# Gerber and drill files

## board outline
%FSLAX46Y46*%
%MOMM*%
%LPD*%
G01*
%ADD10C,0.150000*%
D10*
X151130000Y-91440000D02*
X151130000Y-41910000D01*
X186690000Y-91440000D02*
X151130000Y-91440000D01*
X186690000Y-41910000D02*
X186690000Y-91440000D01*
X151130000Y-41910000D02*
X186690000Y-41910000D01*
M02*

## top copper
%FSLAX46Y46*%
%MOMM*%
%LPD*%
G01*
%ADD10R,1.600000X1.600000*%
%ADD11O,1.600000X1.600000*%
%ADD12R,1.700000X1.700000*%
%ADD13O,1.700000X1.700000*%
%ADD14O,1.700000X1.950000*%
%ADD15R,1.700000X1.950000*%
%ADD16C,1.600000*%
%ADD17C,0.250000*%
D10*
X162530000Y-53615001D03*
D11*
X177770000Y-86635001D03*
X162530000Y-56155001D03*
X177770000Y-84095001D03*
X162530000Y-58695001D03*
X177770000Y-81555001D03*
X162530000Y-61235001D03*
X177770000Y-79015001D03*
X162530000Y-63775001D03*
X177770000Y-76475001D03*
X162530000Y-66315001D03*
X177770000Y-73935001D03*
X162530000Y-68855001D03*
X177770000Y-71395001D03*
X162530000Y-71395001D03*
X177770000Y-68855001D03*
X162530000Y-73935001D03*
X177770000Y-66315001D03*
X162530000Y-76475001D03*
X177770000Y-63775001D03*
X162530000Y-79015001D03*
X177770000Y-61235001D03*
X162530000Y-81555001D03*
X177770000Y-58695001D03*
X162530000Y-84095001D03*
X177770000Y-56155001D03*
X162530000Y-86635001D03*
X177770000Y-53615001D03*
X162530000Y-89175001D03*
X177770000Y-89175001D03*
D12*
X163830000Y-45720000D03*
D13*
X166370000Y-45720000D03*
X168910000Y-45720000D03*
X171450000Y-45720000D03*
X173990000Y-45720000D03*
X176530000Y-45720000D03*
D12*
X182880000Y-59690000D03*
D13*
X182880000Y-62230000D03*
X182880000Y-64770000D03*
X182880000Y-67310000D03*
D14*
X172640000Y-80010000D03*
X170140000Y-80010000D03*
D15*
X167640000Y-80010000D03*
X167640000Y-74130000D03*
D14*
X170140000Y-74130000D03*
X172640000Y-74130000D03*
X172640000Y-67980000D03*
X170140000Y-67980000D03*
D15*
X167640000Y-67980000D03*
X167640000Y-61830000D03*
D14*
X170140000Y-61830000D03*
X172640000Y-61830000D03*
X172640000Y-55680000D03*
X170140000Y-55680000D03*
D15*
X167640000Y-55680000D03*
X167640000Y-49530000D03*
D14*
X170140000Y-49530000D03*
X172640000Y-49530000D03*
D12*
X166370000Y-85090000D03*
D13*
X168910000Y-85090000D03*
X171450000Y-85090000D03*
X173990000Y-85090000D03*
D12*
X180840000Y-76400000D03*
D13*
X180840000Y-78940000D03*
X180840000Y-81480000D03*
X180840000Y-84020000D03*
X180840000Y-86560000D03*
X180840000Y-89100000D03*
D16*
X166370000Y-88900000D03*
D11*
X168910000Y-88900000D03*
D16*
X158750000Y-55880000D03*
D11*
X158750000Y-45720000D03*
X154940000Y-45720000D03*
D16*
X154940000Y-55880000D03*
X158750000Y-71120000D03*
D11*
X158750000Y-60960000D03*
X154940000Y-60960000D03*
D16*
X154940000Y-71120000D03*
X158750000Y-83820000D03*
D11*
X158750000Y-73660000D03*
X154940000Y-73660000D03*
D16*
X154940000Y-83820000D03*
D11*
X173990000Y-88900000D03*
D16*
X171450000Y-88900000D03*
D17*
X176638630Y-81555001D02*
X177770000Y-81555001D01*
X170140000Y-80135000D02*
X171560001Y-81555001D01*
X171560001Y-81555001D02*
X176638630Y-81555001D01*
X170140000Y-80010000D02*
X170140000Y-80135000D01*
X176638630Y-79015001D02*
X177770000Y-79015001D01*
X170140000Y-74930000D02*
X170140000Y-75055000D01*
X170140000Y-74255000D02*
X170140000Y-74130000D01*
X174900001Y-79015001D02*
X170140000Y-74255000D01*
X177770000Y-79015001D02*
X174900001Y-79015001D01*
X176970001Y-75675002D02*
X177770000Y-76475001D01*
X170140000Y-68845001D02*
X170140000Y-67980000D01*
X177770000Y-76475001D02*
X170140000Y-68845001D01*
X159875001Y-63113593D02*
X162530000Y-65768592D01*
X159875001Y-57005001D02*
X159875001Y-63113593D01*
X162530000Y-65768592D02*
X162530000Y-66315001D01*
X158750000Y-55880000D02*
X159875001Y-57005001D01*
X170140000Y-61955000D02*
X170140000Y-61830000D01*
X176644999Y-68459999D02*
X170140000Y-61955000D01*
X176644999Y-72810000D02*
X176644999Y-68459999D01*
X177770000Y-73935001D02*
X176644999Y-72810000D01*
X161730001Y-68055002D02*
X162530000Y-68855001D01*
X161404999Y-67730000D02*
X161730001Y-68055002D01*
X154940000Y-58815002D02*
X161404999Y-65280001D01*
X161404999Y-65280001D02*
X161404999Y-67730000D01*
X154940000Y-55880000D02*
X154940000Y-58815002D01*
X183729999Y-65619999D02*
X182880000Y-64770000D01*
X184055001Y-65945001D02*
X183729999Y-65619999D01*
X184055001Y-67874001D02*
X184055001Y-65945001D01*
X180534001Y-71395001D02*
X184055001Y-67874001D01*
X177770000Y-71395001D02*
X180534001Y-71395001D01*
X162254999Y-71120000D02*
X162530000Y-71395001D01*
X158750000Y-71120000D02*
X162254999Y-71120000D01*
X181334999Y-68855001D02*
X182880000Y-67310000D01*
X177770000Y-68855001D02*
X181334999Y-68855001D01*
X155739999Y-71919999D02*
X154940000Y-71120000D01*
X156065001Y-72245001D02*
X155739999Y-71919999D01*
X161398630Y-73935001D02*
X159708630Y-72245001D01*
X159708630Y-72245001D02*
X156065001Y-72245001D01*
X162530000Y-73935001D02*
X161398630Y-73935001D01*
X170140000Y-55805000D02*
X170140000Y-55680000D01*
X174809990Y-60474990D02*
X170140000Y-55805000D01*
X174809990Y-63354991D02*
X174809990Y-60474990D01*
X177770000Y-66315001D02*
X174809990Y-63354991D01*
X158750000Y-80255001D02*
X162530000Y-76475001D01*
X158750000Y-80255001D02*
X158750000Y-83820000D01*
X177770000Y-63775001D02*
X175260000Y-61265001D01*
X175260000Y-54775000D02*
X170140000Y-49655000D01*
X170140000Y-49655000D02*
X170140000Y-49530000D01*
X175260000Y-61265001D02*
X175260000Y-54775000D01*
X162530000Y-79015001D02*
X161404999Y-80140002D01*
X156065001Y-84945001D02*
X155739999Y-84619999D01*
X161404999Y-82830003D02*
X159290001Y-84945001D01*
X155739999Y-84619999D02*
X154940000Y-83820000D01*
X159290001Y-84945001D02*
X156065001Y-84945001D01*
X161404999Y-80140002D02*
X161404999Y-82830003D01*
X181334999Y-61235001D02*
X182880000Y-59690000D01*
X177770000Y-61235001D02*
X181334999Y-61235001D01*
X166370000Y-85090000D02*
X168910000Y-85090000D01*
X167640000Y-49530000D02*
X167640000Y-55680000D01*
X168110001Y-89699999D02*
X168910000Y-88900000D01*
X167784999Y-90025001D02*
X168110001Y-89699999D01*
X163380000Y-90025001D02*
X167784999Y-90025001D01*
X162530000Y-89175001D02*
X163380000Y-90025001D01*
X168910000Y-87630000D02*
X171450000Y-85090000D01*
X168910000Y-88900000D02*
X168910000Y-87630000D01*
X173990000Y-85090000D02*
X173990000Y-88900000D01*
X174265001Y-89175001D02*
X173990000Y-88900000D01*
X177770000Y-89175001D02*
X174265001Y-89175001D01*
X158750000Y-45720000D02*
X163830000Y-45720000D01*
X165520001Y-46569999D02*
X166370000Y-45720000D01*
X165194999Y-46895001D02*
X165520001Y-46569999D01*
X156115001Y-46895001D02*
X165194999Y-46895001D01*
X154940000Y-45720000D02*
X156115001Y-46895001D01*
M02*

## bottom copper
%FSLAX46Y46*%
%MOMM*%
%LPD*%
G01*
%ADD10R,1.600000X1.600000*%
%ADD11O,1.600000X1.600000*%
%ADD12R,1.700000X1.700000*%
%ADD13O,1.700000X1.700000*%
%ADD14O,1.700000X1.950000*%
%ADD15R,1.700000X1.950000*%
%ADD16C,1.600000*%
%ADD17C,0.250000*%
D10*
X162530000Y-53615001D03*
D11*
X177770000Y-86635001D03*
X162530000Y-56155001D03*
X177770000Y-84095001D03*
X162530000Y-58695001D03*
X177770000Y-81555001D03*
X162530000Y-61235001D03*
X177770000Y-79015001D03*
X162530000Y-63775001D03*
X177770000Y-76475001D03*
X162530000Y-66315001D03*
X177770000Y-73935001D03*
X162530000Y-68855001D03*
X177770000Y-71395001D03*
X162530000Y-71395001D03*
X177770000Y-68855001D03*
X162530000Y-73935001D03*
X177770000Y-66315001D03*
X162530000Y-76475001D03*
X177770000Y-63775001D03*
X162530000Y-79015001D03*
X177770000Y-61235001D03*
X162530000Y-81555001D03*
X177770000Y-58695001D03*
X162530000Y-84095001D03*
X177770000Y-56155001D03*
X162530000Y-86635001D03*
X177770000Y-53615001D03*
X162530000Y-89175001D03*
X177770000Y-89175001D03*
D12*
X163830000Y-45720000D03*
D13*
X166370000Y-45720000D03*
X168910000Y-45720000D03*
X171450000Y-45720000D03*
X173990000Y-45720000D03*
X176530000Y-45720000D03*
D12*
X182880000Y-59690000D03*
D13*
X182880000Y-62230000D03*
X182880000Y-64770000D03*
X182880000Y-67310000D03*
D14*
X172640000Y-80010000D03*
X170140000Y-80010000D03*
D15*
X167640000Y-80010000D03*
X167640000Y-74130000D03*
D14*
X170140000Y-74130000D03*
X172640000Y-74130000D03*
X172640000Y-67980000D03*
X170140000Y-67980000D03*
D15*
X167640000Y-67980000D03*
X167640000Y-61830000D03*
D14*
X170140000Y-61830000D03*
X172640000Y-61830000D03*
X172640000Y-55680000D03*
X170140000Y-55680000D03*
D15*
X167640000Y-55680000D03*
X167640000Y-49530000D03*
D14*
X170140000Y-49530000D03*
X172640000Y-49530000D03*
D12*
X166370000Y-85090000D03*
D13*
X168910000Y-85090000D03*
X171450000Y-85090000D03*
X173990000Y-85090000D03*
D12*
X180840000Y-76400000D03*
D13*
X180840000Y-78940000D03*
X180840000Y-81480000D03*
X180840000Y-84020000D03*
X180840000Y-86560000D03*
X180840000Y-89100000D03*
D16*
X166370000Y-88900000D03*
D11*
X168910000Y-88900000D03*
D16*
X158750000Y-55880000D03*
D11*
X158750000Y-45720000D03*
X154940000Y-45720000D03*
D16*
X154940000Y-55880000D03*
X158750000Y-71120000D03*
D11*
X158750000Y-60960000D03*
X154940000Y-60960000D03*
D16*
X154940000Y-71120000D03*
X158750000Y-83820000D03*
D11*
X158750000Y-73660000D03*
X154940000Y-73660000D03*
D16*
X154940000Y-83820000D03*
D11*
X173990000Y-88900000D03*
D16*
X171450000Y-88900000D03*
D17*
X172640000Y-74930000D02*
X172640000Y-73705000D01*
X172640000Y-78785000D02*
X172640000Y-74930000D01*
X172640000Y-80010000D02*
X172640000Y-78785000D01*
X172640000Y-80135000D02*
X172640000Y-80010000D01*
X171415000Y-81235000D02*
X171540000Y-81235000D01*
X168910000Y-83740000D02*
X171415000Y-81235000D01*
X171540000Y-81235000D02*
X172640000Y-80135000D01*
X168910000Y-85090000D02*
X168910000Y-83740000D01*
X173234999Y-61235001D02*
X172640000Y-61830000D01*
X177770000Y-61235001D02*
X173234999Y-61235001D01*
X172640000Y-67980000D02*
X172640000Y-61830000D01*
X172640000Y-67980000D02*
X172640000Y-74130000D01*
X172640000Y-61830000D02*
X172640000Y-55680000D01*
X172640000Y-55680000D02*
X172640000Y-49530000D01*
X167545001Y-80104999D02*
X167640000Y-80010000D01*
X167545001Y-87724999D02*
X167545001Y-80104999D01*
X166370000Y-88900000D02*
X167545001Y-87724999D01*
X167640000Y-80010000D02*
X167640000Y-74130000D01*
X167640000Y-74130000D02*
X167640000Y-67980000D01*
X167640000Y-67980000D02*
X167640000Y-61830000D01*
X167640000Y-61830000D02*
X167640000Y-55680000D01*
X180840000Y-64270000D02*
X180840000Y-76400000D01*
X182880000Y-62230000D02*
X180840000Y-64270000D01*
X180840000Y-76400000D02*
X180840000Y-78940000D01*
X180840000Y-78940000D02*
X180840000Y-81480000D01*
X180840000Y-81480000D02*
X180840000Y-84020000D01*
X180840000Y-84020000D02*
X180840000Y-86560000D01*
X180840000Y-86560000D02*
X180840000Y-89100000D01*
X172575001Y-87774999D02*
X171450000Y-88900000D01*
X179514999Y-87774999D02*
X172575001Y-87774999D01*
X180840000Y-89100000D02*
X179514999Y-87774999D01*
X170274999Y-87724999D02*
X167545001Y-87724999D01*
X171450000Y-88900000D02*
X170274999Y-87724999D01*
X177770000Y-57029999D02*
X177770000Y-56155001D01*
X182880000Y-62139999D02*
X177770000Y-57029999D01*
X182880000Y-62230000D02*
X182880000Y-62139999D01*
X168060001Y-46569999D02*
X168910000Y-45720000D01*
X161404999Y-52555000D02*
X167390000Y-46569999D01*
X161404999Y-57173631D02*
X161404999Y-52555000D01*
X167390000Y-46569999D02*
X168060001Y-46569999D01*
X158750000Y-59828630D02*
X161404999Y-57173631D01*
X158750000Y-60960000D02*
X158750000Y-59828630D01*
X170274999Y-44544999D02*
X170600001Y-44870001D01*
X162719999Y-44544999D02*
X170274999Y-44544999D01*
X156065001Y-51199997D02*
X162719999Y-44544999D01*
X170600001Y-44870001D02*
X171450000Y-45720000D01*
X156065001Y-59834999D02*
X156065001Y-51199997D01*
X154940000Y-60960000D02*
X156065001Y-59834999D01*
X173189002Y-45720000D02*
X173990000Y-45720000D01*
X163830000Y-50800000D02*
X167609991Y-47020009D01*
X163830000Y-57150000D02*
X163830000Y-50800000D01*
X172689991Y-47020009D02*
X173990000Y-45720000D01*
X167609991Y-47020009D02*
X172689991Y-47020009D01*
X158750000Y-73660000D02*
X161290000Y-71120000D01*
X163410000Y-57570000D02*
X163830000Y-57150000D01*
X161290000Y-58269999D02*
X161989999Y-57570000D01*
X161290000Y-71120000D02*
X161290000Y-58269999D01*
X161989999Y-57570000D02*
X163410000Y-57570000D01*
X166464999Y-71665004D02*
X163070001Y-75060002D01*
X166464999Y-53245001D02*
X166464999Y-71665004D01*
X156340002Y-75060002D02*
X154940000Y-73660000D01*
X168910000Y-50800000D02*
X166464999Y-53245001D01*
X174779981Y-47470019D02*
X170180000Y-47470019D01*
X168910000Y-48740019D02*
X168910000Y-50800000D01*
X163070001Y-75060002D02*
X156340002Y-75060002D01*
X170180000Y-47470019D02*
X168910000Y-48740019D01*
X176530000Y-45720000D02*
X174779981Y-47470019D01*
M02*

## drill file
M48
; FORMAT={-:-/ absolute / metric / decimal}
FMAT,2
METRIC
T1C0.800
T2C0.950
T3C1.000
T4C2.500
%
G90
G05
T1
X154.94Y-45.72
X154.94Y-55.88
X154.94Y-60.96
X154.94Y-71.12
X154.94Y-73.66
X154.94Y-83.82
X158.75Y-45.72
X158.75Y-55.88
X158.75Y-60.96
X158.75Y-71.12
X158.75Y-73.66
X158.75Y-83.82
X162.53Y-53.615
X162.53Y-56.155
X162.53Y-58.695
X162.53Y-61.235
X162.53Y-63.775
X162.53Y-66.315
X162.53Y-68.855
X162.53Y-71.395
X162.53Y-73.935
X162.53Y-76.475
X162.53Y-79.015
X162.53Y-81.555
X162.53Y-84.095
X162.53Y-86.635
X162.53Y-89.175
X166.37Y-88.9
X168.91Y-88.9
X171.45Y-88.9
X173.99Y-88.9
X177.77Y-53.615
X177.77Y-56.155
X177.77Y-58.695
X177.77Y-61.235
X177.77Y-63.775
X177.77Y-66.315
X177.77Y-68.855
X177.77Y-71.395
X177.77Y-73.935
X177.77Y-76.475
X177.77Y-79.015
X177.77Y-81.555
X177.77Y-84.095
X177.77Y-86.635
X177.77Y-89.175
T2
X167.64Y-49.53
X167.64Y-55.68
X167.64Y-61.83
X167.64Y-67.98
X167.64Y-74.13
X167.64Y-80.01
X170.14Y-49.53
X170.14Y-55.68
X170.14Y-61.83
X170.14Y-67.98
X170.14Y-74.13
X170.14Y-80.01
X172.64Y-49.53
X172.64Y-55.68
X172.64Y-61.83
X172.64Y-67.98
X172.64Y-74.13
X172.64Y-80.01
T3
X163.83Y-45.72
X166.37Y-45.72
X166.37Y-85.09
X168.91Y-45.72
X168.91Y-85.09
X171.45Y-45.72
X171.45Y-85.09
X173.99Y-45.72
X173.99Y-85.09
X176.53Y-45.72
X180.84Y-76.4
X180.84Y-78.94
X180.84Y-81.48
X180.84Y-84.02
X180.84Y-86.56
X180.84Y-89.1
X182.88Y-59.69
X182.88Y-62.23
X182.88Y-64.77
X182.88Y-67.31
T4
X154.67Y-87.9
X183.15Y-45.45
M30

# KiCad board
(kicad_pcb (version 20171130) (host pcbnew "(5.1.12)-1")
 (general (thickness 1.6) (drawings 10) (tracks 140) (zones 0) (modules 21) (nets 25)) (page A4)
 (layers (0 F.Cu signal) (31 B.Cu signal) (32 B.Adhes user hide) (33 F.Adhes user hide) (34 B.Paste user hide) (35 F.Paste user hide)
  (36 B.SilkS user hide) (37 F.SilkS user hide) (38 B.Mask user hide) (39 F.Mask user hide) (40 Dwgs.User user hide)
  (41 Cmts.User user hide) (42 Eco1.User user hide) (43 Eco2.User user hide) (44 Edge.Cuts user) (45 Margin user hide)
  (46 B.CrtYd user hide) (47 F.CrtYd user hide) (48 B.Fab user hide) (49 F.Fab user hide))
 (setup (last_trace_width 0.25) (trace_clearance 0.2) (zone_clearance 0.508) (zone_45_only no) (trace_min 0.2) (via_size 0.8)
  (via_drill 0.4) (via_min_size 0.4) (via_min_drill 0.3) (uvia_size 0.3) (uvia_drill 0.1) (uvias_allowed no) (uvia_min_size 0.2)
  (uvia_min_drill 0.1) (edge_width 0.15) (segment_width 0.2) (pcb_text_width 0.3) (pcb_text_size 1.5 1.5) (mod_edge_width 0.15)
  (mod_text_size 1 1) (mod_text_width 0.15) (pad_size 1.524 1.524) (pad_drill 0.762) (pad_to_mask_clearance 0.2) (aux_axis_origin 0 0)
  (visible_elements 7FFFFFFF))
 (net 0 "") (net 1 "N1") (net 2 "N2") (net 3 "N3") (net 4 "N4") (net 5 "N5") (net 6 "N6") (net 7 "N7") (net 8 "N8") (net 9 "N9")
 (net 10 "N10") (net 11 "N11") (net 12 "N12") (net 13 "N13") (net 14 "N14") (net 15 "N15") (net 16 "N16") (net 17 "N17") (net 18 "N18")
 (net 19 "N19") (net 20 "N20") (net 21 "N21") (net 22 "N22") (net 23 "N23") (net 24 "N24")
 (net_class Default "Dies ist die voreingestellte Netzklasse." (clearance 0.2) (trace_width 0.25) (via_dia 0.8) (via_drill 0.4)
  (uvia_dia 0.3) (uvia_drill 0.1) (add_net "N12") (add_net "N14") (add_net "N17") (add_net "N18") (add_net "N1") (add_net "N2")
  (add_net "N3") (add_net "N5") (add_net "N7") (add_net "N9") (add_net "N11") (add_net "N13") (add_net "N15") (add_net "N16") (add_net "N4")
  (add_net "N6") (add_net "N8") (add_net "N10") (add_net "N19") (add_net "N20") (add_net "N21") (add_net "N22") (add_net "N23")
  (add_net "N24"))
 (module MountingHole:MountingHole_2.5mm (layer F.Cu) (at 154.67 87.9)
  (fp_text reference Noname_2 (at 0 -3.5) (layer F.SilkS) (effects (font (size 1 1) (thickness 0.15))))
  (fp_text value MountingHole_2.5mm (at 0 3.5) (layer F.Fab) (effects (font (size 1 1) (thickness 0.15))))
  (pad 1 np_thru_hole circle (at 0 0) (size 2.5 2.5) (drill 2.5) (layers *.Cu *.Mask)))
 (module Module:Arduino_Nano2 (layer F.Cu) (at 162.53 53.615001)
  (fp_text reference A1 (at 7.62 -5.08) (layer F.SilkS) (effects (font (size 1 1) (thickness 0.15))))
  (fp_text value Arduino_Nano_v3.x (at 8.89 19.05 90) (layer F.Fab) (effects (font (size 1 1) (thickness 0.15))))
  (pad 1 thru_hole rect (at 0 0) (size 1.6 1.6) (drill 0.8) (layers *.Cu *.Mask))
  (pad 17 thru_hole oval (at 15.24 33.02) (size 1.6 1.6) (drill 0.8) (layers *.Cu *.Mask))
  (pad 2 thru_hole oval (at 0 2.54) (size 1.6 1.6) (drill 0.8) (layers *.Cu *.Mask))
  (pad 18 thru_hole oval (at 15.24 30.48) (size 1.6 1.6) (drill 0.8) (layers *.Cu *.Mask))
  (pad 3 thru_hole oval (at 0 5.08) (size 1.6 1.6) (drill 0.8) (layers *.Cu *.Mask))
  (pad 19 thru_hole oval (at 15.24 27.94) (size 1.6 1.6) (drill 0.8) (layers *.Cu *.Mask) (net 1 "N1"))
  (pad 4 thru_hole oval (at 0 7.62) (size 1.6 1.6) (drill 0.8) (layers *.Cu *.Mask))
  (pad 20 thru_hole oval (at 15.24 25.4) (size 1.6 1.6) (drill 0.8) (layers *.Cu *.Mask) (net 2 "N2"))
  (pad 5 thru_hole oval (at 0 10.16) (size 1.6 1.6) (drill 0.8) (layers *.Cu *.Mask))
  (pad 21 thru_hole oval (at 15.24 22.86) (size 1.6 1.6) (drill 0.8) (layers *.Cu *.Mask) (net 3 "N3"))
  (pad 6 thru_hole oval (at 0 12.7) (size 1.6 1.6) (drill 0.8) (layers *.Cu *.Mask) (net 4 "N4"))
  (pad 22 thru_hole oval (at 15.24 20.32) (size 1.6 1.6) (drill 0.8) (layers *.Cu *.Mask) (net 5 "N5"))
  (pad 7 thru_hole oval (at 0 15.24) (size 1.6 1.6) (drill 0.8) (layers *.Cu *.Mask) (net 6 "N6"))
  (pad 23 thru_hole oval (at 15.24 17.78) (size 1.6 1.6) (drill 0.8) (layers *.Cu *.Mask) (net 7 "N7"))
  (pad 8 thru_hole oval (at 0 17.78) (size 1.6 1.6) (drill 0.8) (layers *.Cu *.Mask) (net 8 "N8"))
  (pad 24 thru_hole oval (at 15.24 15.24) (size 1.6 1.6) (drill 0.8) (layers *.Cu *.Mask) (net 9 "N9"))
  (pad 9 thru_hole oval (at 0 20.32) (size 1.6 1.6) (drill 0.8) (layers *.Cu *.Mask) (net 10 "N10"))
  (pad 25 thru_hole oval (at 15.24 12.7) (size 1.6 1.6) (drill 0.8) (layers *.Cu *.Mask) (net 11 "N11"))
  (pad 10 thru_hole oval (at 0 22.86) (size 1.6 1.6) (drill 0.8) (layers *.Cu *.Mask) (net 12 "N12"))
  (pad 26 thru_hole oval (at 15.24 10.16) (size 1.6 1.6) (drill 0.8) (layers *.Cu *.Mask) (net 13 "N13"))
  (pad 11 thru_hole oval (at 0 25.4) (size 1.6 1.6) (drill 0.8) (layers *.Cu *.Mask) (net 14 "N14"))
  (pad 27 thru_hole oval (at 15.24 7.62) (size 1.6 1.6) (drill 0.8) (layers *.Cu *.Mask) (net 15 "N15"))
  (pad 12 thru_hole oval (at 0 27.94) (size 1.6 1.6) (drill 0.8) (layers *.Cu *.Mask))
  (pad 28 thru_hole oval (at 15.24 5.08) (size 1.6 1.6) (drill 0.8) (layers *.Cu *.Mask))
  (pad 13 thru_hole oval (at 0 30.48) (size 1.6 1.6) (drill 0.8) (layers *.Cu *.Mask))
  (pad 29 thru_hole oval (at 15.24 2.54) (size 1.6 1.6) (drill 0.8) (layers *.Cu *.Mask) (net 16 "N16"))
  (pad 14 thru_hole oval (at 0 33.02) (size 1.6 1.6) (drill 0.8) (layers *.Cu *.Mask))
  (pad 30 thru_hole oval (at 15.24 0) (size 1.6 1.6) (drill 0.8) (layers *.Cu *.Mask))
  (pad 15 thru_hole oval (at 0 35.56) (size 1.6 1.6) (drill 0.8) (layers *.Cu *.Mask) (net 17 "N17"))
  (pad 16 thru_hole oval (at 15.24 35.56) (size 1.6 1.6) (drill 0.8) (layers *.Cu *.Mask) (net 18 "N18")))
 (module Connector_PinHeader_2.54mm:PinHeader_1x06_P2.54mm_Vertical (layer F.Cu) (at 163.83 45.72 90)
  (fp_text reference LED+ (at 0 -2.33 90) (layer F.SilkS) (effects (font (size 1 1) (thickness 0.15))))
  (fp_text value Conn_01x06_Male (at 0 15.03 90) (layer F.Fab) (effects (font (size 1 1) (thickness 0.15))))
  (pad 1 thru_hole rect (at 0 0 90) (size 1.7 1.7) (drill 1) (layers *.Cu *.Mask) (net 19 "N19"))
  (pad 2 thru_hole oval (at 0 2.54 90) (size 1.7 1.7) (drill 1) (layers *.Cu *.Mask) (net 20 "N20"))
  (pad 3 thru_hole oval (at 0 5.08 90) (size 1.7 1.7) (drill 1) (layers *.Cu *.Mask) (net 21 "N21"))
  (pad 4 thru_hole oval (at 0 7.62 90) (size 1.7 1.7) (drill 1) (layers *.Cu *.Mask) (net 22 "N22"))
  (pad 5 thru_hole oval (at 0 10.16 90) (size 1.7 1.7) (drill 1) (layers *.Cu *.Mask) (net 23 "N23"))
  (pad 6 thru_hole oval (at 0 12.7 90) (size 1.7 1.7) (drill 1) (layers *.Cu *.Mask) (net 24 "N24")))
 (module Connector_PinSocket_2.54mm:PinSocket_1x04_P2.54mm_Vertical (layer F.Cu) (at 182.88 59.69)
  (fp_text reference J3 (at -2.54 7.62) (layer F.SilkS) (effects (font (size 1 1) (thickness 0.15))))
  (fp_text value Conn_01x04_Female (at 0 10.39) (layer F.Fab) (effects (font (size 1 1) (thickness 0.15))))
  (pad 1 thru_hole rect (at 0 0) (size 1.7 1.7) (drill 1) (layers *.Cu *.Mask) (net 15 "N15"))
  (pad 2 thru_hole oval (at 0 2.54) (size 1.7 1.7) (drill 1) (layers *.Cu *.Mask) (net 16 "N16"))
  (pad 3 thru_hole oval (at 0 5.08) (size 1.7 1.7) (drill 1) (layers *.Cu *.Mask) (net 7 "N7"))
  (pad 4 thru_hole oval (at 0 7.62) (size 1.7 1.7) (drill 1) (layers *.Cu *.Mask) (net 9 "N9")))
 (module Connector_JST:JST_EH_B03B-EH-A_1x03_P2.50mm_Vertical (layer F.Cu) (at 167.64 80.01)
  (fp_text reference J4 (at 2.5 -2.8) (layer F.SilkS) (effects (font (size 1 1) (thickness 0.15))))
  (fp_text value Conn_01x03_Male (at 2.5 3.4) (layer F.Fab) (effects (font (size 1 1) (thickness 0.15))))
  (pad 3 thru_hole oval (at 5 0) (size 1.7 1.95) (drill 0.95) (layers *.Cu *.Mask) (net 15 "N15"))
  (pad 2 thru_hole oval (at 2.5 0) (size 1.7 1.95) (drill 0.95) (layers *.Cu *.Mask) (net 1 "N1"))
  (pad 1 thru_hole rect (at 0 0) (size 1.7 1.95) (drill 0.95) (layers *.Cu *.Mask) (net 16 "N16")))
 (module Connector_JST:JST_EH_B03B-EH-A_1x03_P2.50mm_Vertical (layer F.Cu) (at 167.64 74.13)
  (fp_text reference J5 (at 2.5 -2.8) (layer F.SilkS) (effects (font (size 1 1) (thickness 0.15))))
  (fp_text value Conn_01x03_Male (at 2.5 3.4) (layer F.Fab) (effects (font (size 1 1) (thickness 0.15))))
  (pad 1 thru_hole rect (at 0 0) (size 1.7 1.95) (drill 0.95) (layers *.Cu *.Mask) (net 16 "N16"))
  (pad 2 thru_hole oval (at 2.5 0) (size 1.7 1.95) (drill 0.95) (layers *.Cu *.Mask) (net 2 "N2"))
  (pad 3 thru_hole oval (at 5 0) (size 1.7 1.95) (drill 0.95) (layers *.Cu *.Mask) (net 15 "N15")))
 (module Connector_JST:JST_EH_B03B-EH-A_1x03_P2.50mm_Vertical (layer F.Cu) (at 167.64 67.98)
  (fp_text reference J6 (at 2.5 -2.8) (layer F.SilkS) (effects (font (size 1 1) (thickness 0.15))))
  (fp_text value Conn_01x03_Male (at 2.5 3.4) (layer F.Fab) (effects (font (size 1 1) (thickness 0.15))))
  (pad 3 thru_hole oval (at 5 0) (size 1.7 1.95) (drill 0.95) (layers *.Cu *.Mask) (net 15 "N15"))
  (pad 2 thru_hole oval (at 2.5 0) (size 1.7 1.95) (drill 0.95) (layers *.Cu *.Mask) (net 3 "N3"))
  (pad 1 thru_hole rect (at 0 0) (size 1.7 1.95) (drill 0.95) (layers *.Cu *.Mask) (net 16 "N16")))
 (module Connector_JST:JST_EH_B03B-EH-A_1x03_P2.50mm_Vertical (layer F.Cu) (at 167.64 61.83)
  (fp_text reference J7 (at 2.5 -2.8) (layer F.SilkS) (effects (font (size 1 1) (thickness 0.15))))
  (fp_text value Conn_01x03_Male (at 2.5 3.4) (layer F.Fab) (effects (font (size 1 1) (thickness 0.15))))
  (pad 1 thru_hole rect (at 0 0) (size 1.7 1.95) (drill 0.95) (layers *.Cu *.Mask) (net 16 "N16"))
  (pad 2 thru_hole oval (at 2.5 0) (size 1.7 1.95) (drill 0.95) (layers *.Cu *.Mask) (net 5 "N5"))
  (pad 3 thru_hole oval (at 5 0) (size 1.7 1.95) (drill 0.95) (layers *.Cu *.Mask) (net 15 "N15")))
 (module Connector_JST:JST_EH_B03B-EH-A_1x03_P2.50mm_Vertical (layer F.Cu) (at 167.64 55.68)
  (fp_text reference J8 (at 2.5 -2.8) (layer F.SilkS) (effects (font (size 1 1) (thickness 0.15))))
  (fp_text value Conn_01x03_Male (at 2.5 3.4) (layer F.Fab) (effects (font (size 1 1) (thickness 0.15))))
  (pad 3 thru_hole oval (at 5 0) (size 1.7 1.95) (drill 0.95) (layers *.Cu *.Mask) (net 15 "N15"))
  (pad 2 thru_hole oval (at 2.5 0) (size 1.7 1.95) (drill 0.95) (layers *.Cu *.Mask) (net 11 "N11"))
  (pad 1 thru_hole rect (at 0 0) (size 1.7 1.95) (drill 0.95) (layers *.Cu *.Mask) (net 16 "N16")))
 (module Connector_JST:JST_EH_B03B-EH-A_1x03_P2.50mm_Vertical (layer F.Cu) (at 167.64 49.53)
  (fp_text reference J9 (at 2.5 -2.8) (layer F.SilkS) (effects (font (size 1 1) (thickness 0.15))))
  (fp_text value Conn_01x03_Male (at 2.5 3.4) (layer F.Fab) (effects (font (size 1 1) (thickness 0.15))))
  (pad 1 thru_hole rect (at 0 0) (size 1.7 1.95) (drill 0.95) (layers *.Cu *.Mask) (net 16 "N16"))
  (pad 2 thru_hole oval (at 2.5 0) (size 1.7 1.95) (drill 0.95) (layers *.Cu *.Mask) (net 13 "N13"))
  (pad 3 thru_hole oval (at 5 0) (size 1.7 1.95) (drill 0.95) (layers *.Cu *.Mask) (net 15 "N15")))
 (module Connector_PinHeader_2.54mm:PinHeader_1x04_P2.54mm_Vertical (layer F.Cu) (at 166.37 85.09 90)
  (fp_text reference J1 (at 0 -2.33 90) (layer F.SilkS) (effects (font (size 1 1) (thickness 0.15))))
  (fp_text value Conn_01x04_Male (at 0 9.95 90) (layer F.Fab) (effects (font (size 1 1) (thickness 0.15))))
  (pad 1 thru_hole rect (at 0 0 90) (size 1.7 1.7) (drill 1) (layers *.Cu *.Mask) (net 15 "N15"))
  (pad 2 thru_hole oval (at 0 2.54 90) (size 1.7 1.7) (drill 1) (layers *.Cu *.Mask) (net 15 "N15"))
  (pad 3 thru_hole oval (at 0 5.08 90) (size 1.7 1.7) (drill 1) (layers *.Cu *.Mask) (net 17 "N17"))
  (pad 4 thru_hole oval (at 0 7.62 90) (size 1.7 1.7) (drill 1) (layers *.Cu *.Mask) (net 18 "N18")))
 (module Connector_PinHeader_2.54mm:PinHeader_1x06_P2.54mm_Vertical (layer F.Cu) (at 180.84 76.4)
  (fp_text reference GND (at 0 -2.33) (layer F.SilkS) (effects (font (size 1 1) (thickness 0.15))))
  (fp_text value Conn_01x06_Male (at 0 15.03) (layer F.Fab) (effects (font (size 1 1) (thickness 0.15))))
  (pad 1 thru_hole rect (at 0 0) (size 1.7 1.7) (drill 1) (layers *.Cu *.Mask) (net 16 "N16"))
  (pad 2 thru_hole oval (at 0 2.54) (size 1.7 1.7) (drill 1) (layers *.Cu *.Mask) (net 16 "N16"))
  (pad 3 thru_hole oval (at 0 5.08) (size 1.7 1.7) (drill 1) (layers *.Cu *.Mask) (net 16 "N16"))
  (pad 4 thru_hole oval (at 0 7.62) (size 1.7 1.7) (drill 1) (layers *.Cu *.Mask) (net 16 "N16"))
  (pad 5 thru_hole oval (at 0 10.16) (size 1.7 1.7) (drill 1) (layers *.Cu *.Mask) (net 16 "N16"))
  (pad 6 thru_hole oval (at 0 12.7) (size 1.7 1.7) (drill 1) (layers *.Cu *.Mask) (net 16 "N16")))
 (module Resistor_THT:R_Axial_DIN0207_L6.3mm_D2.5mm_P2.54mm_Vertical (layer F.Cu) (at 166.37 88.9)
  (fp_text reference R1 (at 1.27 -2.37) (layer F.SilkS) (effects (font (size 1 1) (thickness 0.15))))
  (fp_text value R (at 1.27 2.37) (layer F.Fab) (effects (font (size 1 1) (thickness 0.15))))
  (pad 1 thru_hole circle (at 0 0) (size 1.6 1.6) (drill 0.8) (layers *.Cu *.Mask) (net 16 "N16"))
  (pad 2 thru_hole oval (at 2.54 0) (size 1.6 1.6) (drill 0.8) (layers *.Cu *.Mask) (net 17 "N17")))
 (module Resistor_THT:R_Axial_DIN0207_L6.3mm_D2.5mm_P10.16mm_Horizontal (layer F.Cu) (at 158.75 55.88 90)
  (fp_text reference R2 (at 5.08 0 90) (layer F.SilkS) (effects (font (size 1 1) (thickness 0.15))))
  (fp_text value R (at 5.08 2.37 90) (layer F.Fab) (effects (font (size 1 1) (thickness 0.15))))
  (pad 1 thru_hole circle (at 0 0 90) (size 1.6 1.6) (drill 0.8) (layers *.Cu *.Mask) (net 4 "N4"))
  (pad 2 thru_hole oval (at 10.16 0 90) (size 1.6 1.6) (drill 0.8) (layers *.Cu *.Mask) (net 19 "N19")))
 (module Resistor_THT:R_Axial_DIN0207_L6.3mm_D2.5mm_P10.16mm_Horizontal (layer F.Cu) (at 154.94 55.88 90)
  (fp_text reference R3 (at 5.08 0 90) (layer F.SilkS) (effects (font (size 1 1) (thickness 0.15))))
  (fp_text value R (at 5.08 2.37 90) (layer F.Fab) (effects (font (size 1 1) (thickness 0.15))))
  (pad 2 thru_hole oval (at 10.16 0 90) (size 1.6 1.6) (drill 0.8) (layers *.Cu *.Mask) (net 20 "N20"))
  (pad 1 thru_hole circle (at 0 0 90) (size 1.6 1.6) (drill 0.8) (layers *.Cu *.Mask) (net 6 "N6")))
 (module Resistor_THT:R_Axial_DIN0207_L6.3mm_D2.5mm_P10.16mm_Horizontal (layer F.Cu) (at 158.75 71.12 90)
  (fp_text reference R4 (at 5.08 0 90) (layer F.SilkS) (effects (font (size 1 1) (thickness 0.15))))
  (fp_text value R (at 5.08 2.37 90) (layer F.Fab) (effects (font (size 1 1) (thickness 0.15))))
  (pad 1 thru_hole circle (at 0 0 90) (size 1.6 1.6) (drill 0.8) (layers *.Cu *.Mask) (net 8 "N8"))
  (pad 2 thru_hole oval (at 10.16 0 90) (size 1.6 1.6) (drill 0.8) (layers *.Cu *.Mask) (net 21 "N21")))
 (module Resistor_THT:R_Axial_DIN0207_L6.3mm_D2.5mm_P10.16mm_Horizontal (layer F.Cu) (at 154.94 71.12 90)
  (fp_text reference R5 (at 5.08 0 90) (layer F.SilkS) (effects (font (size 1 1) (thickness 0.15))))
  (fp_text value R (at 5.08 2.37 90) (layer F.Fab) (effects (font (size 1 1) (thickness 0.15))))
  (pad 2 thru_hole oval (at 10.16 0 90) (size 1.6 1.6) (drill 0.8) (layers *.Cu *.Mask) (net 22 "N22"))
  (pad 1 thru_hole circle (at 0 0 90) (size 1.6 1.6) (drill 0.8) (layers *.Cu *.Mask) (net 10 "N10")))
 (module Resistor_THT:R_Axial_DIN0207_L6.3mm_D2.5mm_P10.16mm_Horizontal (layer F.Cu) (at 158.75 83.82 90)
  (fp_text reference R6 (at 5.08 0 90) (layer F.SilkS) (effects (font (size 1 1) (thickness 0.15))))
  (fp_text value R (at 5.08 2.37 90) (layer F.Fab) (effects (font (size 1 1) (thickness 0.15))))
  (pad 1 thru_hole circle (at 0 0 90) (size 1.6 1.6) (drill 0.8) (layers *.Cu *.Mask) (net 12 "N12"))
  (pad 2 thru_hole oval (at 10.16 0 90) (size 1.6 1.6) (drill 0.8) (layers *.Cu *.Mask) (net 23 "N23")))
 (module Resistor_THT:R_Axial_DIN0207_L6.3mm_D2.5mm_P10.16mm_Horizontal (layer F.Cu) (at 154.94 83.82 90)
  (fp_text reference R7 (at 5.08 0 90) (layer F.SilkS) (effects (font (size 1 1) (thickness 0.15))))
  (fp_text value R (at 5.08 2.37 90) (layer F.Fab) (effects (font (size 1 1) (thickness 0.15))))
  (pad 2 thru_hole oval (at 10.16 0 90) (size 1.6 1.6) (drill 0.8) (layers *.Cu *.Mask) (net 24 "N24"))
  (pad 1 thru_hole circle (at 0 0 90) (size 1.6 1.6) (drill 0.8) (layers *.Cu *.Mask) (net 14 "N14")))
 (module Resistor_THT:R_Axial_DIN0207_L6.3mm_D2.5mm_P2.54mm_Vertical (layer F.Cu) (at 171.45 88.9)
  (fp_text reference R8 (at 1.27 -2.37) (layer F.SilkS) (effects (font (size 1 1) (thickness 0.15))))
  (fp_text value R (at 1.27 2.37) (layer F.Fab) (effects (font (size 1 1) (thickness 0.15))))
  (pad 2 thru_hole oval (at 2.54 0) (size 1.6 1.6) (drill 0.8) (layers *.Cu *.Mask) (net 18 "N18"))
  (pad 1 thru_hole circle (at 0 0) (size 1.6 1.6) (drill 0.8) (layers *.Cu *.Mask) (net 16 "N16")))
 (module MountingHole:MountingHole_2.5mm (layer F.Cu) (at 183.15 45.45)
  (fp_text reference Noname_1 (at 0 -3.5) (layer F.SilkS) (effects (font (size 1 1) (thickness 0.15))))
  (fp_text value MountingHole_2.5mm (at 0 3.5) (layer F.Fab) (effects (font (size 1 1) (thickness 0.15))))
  (pad 1 np_thru_hole circle (at 0 0) (size 2.5 2.5) (drill 2.5) (layers *.Cu *.Mask)))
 (gr_line (start 151.13 91.44) (end 151.13 41.91) (layer Edge.Cuts) (width 0.15))
 (gr_line (start 186.69 91.44) (end 151.13 91.44) (layer Edge.Cuts) (width 0.15))
 (gr_line (start 186.69 41.91) (end 186.69 91.44) (layer Edge.Cuts) (width 0.15))
 (gr_line (start 151.13 41.91) (end 186.69 41.91) (layer Edge.Cuts) (width 0.15))
 (segment (start 176.63863 81.555001) (end 177.77 81.555001) (width 0.25) (layer F.Cu) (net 1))
 (segment (start 170.14 80.135) (end 171.560001 81.555001) (width 0.25) (layer F.Cu) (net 1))
 (segment (start 171.560001 81.555001) (end 176.63863 81.555001) (width 0.25) (layer F.Cu) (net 1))
 (segment (start 170.14 80.01) (end 170.14 80.135) (width 0.25) (layer F.Cu) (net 1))
 (segment (start 176.63863 79.015001) (end 177.77 79.015001) (width 0.25) (layer F.Cu) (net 2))
 (segment (start 170.14 74.93) (end 170.14 75.055) (width 0.25) (layer F.Cu) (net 2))
 (segment (start 170.14 74.255) (end 170.14 74.13) (width 0.25) (layer F.Cu) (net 2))
 (segment (start 174.900001 79.015001) (end 170.14 74.255) (width 0.25) (layer F.Cu) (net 2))
 (segment (start 177.77 79.015001) (end 174.900001 79.015001) (width 0.25) (layer F.Cu) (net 2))
 (segment (start 176.970001 75.675002) (end 177.77 76.475001) (width 0.25) (layer F.Cu) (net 3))
 (segment (start 170.14 68.845001) (end 170.14 67.98) (width 0.25) (layer F.Cu) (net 3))
 (segment (start 177.77 76.475001) (end 170.14 68.845001) (width 0.25) (layer F.Cu) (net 3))
 (segment (start 159.875001 63.113593) (end 162.53 65.768592) (width 0.25) (layer F.Cu) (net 4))
 (segment (start 159.875001 57.005001) (end 159.875001 63.113593) (width 0.25) (layer F.Cu) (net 4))
 (segment (start 162.53 65.768592) (end 162.53 66.315001) (width 0.25) (layer F.Cu) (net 4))
 (segment (start 158.75 55.88) (end 159.875001 57.005001) (width 0.25) (layer F.Cu) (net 4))
 (segment (start 170.14 61.955) (end 170.14 61.83) (width 0.25) (layer F.Cu) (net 5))
 (segment (start 176.644999 68.459999) (end 170.14 61.955) (width 0.25) (layer F.Cu) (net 5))
 (segment (start 176.644999 72.81) (end 176.644999 68.459999) (width 0.25) (layer F.Cu) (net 5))
 (segment (start 177.77 73.935001) (end 176.644999 72.81) (width 0.25) (layer F.Cu) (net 5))
 (segment (start 161.730001 68.055002) (end 162.53 68.855001) (width 0.25) (layer F.Cu) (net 6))
 (segment (start 161.404999 67.73) (end 161.730001 68.055002) (width 0.25) (layer F.Cu) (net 6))
 (segment (start 154.94 58.815002) (end 161.404999 65.280001) (width 0.25) (layer F.Cu) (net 6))
 (segment (start 161.404999 65.280001) (end 161.404999 67.73) (width 0.25) (layer F.Cu) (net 6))
 (segment (start 154.94 55.88) (end 154.94 58.815002) (width 0.25) (layer F.Cu) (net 6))
 (segment (start 183.729999 65.619999) (end 182.88 64.77) (width 0.25) (layer F.Cu) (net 7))
 (segment (start 184.055001 65.945001) (end 183.729999 65.619999) (width 0.25) (layer F.Cu) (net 7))
 (segment (start 184.055001 67.874001) (end 184.055001 65.945001) (width 0.25) (layer F.Cu) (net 7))
 (segment (start 180.534001 71.395001) (end 184.055001 67.874001) (width 0.25) (layer F.Cu) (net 7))
 (segment (start 177.77 71.395001) (end 180.534001 71.395001) (width 0.25) (layer F.Cu) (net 7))
 (segment (start 162.254999 71.12) (end 162.53 71.395001) (width 0.25) (layer F.Cu) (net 8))
 (segment (start 158.75 71.12) (end 162.254999 71.12) (width 0.25) (layer F.Cu) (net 8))
 (segment (start 181.334999 68.855001) (end 182.88 67.31) (width 0.25) (layer F.Cu) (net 9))
 (segment (start 177.77 68.855001) (end 181.334999 68.855001) (width 0.25) (layer F.Cu) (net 9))
 (segment (start 155.739999 71.919999) (end 154.94 71.12) (width 0.25) (layer F.Cu) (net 10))
 (segment (start 156.065001 72.245001) (end 155.739999 71.919999) (width 0.25) (layer F.Cu) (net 10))
 (segment (start 161.39863 73.935001) (end 159.70863 72.245001) (width 0.25) (layer F.Cu) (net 10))
 (segment (start 159.70863 72.245001) (end 156.065001 72.245001) (width 0.25) (layer F.Cu) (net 10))
 (segment (start 162.53 73.935001) (end 161.39863 73.935001) (width 0.25) (layer F.Cu) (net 10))
 (segment (start 170.14 55.805) (end 170.14 55.68) (width 0.25) (layer F.Cu) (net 11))
 (segment (start 174.80999 60.47499) (end 170.14 55.805) (width 0.25) (layer F.Cu) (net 11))
 (segment (start 174.80999 63.354991) (end 174.80999 60.47499) (width 0.25) (layer F.Cu) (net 11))
 (segment (start 177.77 66.315001) (end 174.80999 63.354991) (width 0.25) (layer F.Cu) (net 11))
 (segment (start 158.75 80.255001) (end 162.53 76.475001) (width 0.25) (layer F.Cu) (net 12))
 (segment (start 158.75 80.255001) (end 158.75 83.82) (width 0.25) (layer F.Cu) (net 12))
 (segment (start 177.77 63.775001) (end 175.26 61.265001) (width 0.25) (layer F.Cu) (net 13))
 (segment (start 175.26 54.775) (end 170.14 49.655) (width 0.25) (layer F.Cu) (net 13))
 (segment (start 170.14 49.655) (end 170.14 49.53) (width 0.25) (layer F.Cu) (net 13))
 (segment (start 175.26 61.265001) (end 175.26 54.775) (width 0.25) (layer F.Cu) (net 13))
 (segment (start 162.53 79.015001) (end 161.404999 80.140002) (width 0.25) (layer F.Cu) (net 14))
 (segment (start 156.065001 84.945001) (end 155.739999 84.619999) (width 0.25) (layer F.Cu) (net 14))
 (segment (start 161.404999 82.830003) (end 159.290001 84.945001) (width 0.25) (layer F.Cu) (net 14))
 (segment (start 155.739999 84.619999) (end 154.94 83.82) (width 0.25) (layer F.Cu) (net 14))
 (segment (start 159.290001 84.945001) (end 156.065001 84.945001) (width 0.25) (layer F.Cu) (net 14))
 (segment (start 161.404999 80.140002) (end 161.404999 82.830003) (width 0.25) (layer F.Cu) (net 14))
 (segment (start 181.334999 61.235001) (end 182.88 59.69) (width 0.25) (layer F.Cu) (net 15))
 (segment (start 177.77 61.235001) (end 181.334999 61.235001) (width 0.25) (layer F.Cu) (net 15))
 (segment (start 172.64 74.93) (end 172.64 73.705) (width 0.25) (layer B.Cu) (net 15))
 (segment (start 172.64 78.785) (end 172.64 74.93) (width 0.25) (layer B.Cu) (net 15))
 (segment (start 172.64 80.01) (end 172.64 78.785) (width 0.25) (layer B.Cu) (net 15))
 (segment (start 172.64 80.135) (end 172.64 80.01) (width 0.25) (layer B.Cu) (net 15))
 (segment (start 171.415 81.235) (end 171.54 81.235) (width 0.25) (layer B.Cu) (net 15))
 (segment (start 168.91 83.74) (end 171.415 81.235) (width 0.25) (layer B.Cu) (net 15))
 (segment (start 171.54 81.235) (end 172.64 80.135) (width 0.25) (layer B.Cu) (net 15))
 (segment (start 168.91 85.09) (end 168.91 83.74) (width 0.25) (layer B.Cu) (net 15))
 (segment (start 166.37 85.09) (end 168.91 85.09) (width 0.25) (layer F.Cu) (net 15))
 (segment (start 173.234999 61.235001) (end 172.64 61.83) (width 0.25) (layer B.Cu) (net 15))
 (segment (start 177.77 61.235001) (end 173.234999 61.235001) (width 0.25) (layer B.Cu) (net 15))
 (segment (start 172.64 67.98) (end 172.64 61.83) (width 0.25) (layer B.Cu) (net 15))
 (segment (start 172.64 67.98) (end 172.64 74.13) (width 0.25) (layer B.Cu) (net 15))
 (segment (start 172.64 61.83) (end 172.64 55.68) (width 0.25) (layer B.Cu) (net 15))
 (segment (start 172.64 55.68) (end 172.64 49.53) (width 0.25) (layer B.Cu) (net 15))
 (segment (start 167.64 49.53) (end 167.64 55.68) (width 0.25) (layer F.Cu) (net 16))
 (segment (start 167.545001 80.104999) (end 167.64 80.01) (width 0.25) (layer B.Cu) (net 16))
 (segment (start 167.545001 87.724999) (end 167.545001 80.104999) (width 0.25) (layer B.Cu) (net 16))
 (segment (start 166.37 88.9) (end 167.545001 87.724999) (width 0.25) (layer B.Cu) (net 16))
 (segment (start 167.64 80.01) (end 167.64 74.13) (width 0.25) (layer B.Cu) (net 16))
 (segment (start 167.64 74.13) (end 167.64 67.98) (width 0.25) (layer B.Cu) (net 16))
 (segment (start 167.64 67.98) (end 167.64 61.83) (width 0.25) (layer B.Cu) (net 16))
 (segment (start 167.64 61.83) (end 167.64 55.68) (width 0.25) (layer B.Cu) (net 16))
 (segment (start 180.84 64.27) (end 180.84 76.4) (width 0.25) (layer B.Cu) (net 16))
 (segment (start 182.88 62.23) (end 180.84 64.27) (width 0.25) (layer B.Cu) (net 16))
 (segment (start 180.84 76.4) (end 180.84 78.94) (width 0.25) (layer B.Cu) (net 16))
 (segment (start 180.84 78.94) (end 180.84 81.48) (width 0.25) (layer B.Cu) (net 16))
 (segment (start 180.84 81.48) (end 180.84 84.02) (width 0.25) (layer B.Cu) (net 16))
 (segment (start 180.84 84.02) (end 180.84 86.56) (width 0.25) (layer B.Cu) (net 16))
 (segment (start 180.84 86.56) (end 180.84 89.1) (width 0.25) (layer B.Cu) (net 16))
 (segment (start 172.575001 87.774999) (end 171.45 88.9) (width 0.25) (layer B.Cu) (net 16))
 (segment (start 179.514999 87.774999) (end 172.575001 87.774999) (width 0.25) (layer B.Cu) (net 16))
 (segment (start 180.84 89.1) (end 179.514999 87.774999) (width 0.25) (layer B.Cu) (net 16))
 (segment (start 170.274999 87.724999) (end 167.545001 87.724999) (width 0.25) (layer B.Cu) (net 16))
 (segment (start 171.45 88.9) (end 170.274999 87.724999) (width 0.25) (layer B.Cu) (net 16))
 (segment (start 177.77 57.029999) (end 177.77 56.155001) (width 0.25) (layer B.Cu) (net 16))
 (segment (start 182.88 62.139999) (end 177.77 57.029999) (width 0.25) (layer B.Cu) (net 16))
 (segment (start 182.88 62.23) (end 182.88 62.139999) (width 0.25) (layer B.Cu) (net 16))
 (segment (start 168.110001 89.699999) (end 168.91 88.9) (width 0.25) (layer F.Cu) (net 17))
 (segment (start 167.784999 90.025001) (end 168.110001 89.699999) (width 0.25) (layer F.Cu) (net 17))
 (segment (start 163.38 90.025001) (end 167.784999 90.025001) (width 0.25) (layer F.Cu) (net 17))
 (segment (start 162.53 89.175001) (end 163.38 90.025001) (width 0.25) (layer F.Cu) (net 17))
 (segment (start 168.91 87.63) (end 171.45 85.09) (width 0.25) (layer F.Cu) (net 17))
 (segment (start 168.91 88.9) (end 168.91 87.63) (width 0.25) (layer F.Cu) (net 17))
 (segment (start 173.99 85.09) (end 173.99 88.9) (width 0.25) (layer F.Cu) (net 18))
 (segment (start 174.265001 89.175001) (end 173.99 88.9) (width 0.25) (layer F.Cu) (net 18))
 (segment (start 177.77 89.175001) (end 174.265001 89.175001) (width 0.25) (layer F.Cu) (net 18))
 (segment (start 158.75 45.72) (end 163.83 45.72) (width 0.25) (layer F.Cu) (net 19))
 (segment (start 165.520001 46.569999) (end 166.37 45.72) (width 0.25) (layer F.Cu) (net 20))
 (segment (start 165.194999 46.895001) (end 165.520001 46.569999) (width 0.25) (layer F.Cu) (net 20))
 (segment (start 156.115001 46.895001) (end 165.194999 46.895001) (width 0.25) (layer F.Cu) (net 20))
 (segment (start 154.94 45.72) (end 156.115001 46.895001) (width 0.25) (layer F.Cu) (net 20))
 (segment (start 168.060001 46.569999) (end 168.91 45.72) (width 0.25) (layer B.Cu) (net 21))
 (segment (start 161.404999 52.555) (end 167.39 46.569999) (width 0.25) (layer B.Cu) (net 21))
 (segment (start 161.404999 57.173631) (end 161.404999 52.555) (width 0.25) (layer B.Cu) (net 21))
 (segment (start 167.39 46.569999) (end 168.060001 46.569999) (width 0.25) (layer B.Cu) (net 21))
 (segment (start 158.75 59.82863) (end 161.404999 57.173631) (width 0.25) (layer B.Cu) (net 21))
 (segment (start 158.75 60.96) (end 158.75 59.82863) (width 0.25) (layer B.Cu) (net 21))
 (segment (start 170.274999 44.544999) (end 170.600001 44.870001) (width 0.25) (layer B.Cu) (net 22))
 (segment (start 162.719999 44.544999) (end 170.274999 44.544999) (width 0.25) (layer B.Cu) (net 22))
 (segment (start 156.065001 51.199997) (end 162.719999 44.544999) (width 0.25) (layer B.Cu) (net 22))
 (segment (start 170.600001 44.870001) (end 171.45 45.72) (width 0.25) (layer B.Cu) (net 22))
 (segment (start 156.065001 59.834999) (end 156.065001 51.199997) (width 0.25) (layer B.Cu) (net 22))
 (segment (start 154.94 60.96) (end 156.065001 59.834999) (width 0.25) (layer B.Cu) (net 22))
 (segment (start 173.189002 45.72) (end 173.99 45.72) (width 0.25) (layer B.Cu) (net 23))
 (segment (start 163.83 50.8) (end 167.609991 47.020009) (width 0.25) (layer B.Cu) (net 23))
 (segment (start 163.83 57.15) (end 163.83 50.8) (width 0.25) (layer B.Cu) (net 23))
 (segment (start 172.689991 47.020009) (end 173.99 45.72) (width 0.25) (layer B.Cu) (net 23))
 (segment (start 167.609991 47.020009) (end 172.689991 47.020009) (width 0.25) (layer B.Cu) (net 23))
 (segment (start 158.75 73.66) (end 161.29 71.12) (width 0.25) (layer B.Cu) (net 23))
 (segment (start 163.41 57.57) (end 163.83 57.15) (width 0.25) (layer B.Cu) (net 23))
 (segment (start 161.29 58.269999) (end 161.989999 57.57) (width 0.25) (layer B.Cu) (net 23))
 (segment (start 161.29 71.12) (end 161.29 58.269999) (width 0.25) (layer B.Cu) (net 23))
 (segment (start 161.989999 57.57) (end 163.41 57.57) (width 0.25) (layer B.Cu) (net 23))
 (segment (start 166.464999 71.665004) (end 163.070001 75.060002) (width 0.25) (layer B.Cu) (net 24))
 (segment (start 166.464999 53.245001) (end 166.464999 71.665004) (width 0.25) (layer B.Cu) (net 24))
 (segment (start 156.340002 75.060002) (end 154.94 73.66) (width 0.25) (layer B.Cu) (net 24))
 (segment (start 168.91 50.8) (end 166.464999 53.245001) (width 0.25) (layer B.Cu) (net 24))
 (segment (start 174.779981 47.470019) (end 170.18 47.470019) (width 0.25) (layer B.Cu) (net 24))
 (segment (start 168.91 48.740019) (end 168.91 50.8) (width 0.25) (layer B.Cu) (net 24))
 (segment (start 163.070001 75.060002) (end 156.340002 75.060002) (width 0.25) (layer B.Cu) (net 24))
 (segment (start 170.18 47.470019) (end 168.91 48.740019) (width 0.25) (layer B.Cu) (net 24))
 (segment (start 176.53 45.72) (end 174.779981 47.470019) (width 0.25) (layer B.Cu) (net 24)))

